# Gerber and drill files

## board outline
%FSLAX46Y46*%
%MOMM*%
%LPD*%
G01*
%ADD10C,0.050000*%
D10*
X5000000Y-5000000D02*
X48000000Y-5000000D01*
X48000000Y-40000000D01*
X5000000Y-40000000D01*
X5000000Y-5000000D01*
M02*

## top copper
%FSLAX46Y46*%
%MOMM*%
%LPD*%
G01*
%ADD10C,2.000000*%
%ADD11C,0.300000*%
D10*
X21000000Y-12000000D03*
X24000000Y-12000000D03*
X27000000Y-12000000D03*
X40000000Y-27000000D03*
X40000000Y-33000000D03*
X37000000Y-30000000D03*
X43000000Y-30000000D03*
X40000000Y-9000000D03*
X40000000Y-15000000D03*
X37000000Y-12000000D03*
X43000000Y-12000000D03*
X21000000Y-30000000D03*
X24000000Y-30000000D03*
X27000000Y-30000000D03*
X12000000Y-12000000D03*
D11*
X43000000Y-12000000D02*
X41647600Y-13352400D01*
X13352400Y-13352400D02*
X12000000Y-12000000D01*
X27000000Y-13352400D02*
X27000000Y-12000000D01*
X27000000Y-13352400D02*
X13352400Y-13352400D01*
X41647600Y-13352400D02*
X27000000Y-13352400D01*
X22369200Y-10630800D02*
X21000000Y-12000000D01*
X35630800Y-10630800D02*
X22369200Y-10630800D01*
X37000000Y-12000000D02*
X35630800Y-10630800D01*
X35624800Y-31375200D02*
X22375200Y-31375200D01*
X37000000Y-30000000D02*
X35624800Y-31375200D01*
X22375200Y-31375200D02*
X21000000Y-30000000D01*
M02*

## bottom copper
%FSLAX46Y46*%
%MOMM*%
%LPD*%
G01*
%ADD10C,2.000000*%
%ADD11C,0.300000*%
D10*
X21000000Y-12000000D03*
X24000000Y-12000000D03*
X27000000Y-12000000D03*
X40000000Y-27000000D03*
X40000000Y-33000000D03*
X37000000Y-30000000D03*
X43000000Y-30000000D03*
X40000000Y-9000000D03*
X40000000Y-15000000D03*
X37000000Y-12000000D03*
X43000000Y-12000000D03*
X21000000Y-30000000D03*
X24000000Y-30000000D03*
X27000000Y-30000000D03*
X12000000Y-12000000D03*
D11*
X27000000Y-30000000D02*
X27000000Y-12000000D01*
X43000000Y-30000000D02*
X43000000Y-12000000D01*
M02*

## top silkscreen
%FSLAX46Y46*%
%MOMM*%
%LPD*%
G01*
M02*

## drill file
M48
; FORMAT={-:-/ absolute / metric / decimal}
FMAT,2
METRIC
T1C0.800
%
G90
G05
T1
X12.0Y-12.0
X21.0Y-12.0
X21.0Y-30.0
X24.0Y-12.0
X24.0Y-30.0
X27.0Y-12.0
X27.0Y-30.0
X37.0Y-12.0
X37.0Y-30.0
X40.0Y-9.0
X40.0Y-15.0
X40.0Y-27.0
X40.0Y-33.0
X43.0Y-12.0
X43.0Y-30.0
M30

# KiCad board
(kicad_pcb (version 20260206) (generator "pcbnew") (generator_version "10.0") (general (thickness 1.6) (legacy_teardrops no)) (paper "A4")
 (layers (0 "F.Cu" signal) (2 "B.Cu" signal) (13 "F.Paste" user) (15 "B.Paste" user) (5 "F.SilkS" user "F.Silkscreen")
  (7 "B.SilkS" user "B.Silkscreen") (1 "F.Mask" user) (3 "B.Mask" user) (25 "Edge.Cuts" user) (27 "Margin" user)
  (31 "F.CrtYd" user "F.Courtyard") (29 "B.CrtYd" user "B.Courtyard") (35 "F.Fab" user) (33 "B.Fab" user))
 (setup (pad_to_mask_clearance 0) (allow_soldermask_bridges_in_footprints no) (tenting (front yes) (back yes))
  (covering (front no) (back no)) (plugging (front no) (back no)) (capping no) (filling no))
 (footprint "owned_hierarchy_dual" (layer "F.Cu") (at 24 12)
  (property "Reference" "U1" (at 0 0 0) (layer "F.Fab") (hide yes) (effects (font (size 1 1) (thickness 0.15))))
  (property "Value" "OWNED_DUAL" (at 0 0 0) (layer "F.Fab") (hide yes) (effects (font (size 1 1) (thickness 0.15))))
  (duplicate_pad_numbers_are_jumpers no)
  (pad "1" thru_hole circle (at -3 0) (size 2 2) (drill 0.8) (layers "*.Cu" "*.Mask") (remove_unused_layers no) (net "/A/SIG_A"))
  (pad "2" thru_hole circle (at 0 0) (size 2 2) (drill 0.8) (layers "*.Cu" "*.Mask") (remove_unused_layers no) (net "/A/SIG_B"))
  (pad "3" thru_hole circle (at 3 0) (size 2 2) (drill 0.8) (layers "*.Cu" "*.Mask") (remove_unused_layers no) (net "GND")))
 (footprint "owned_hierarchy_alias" (layer "F.Cu") (at 40 30)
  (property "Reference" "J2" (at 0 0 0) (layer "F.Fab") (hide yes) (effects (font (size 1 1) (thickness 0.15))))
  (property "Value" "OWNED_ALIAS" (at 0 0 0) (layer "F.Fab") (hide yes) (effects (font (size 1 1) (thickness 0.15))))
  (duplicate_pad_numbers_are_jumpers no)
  (pad "MP" thru_hole circle (at 0 -3) (size 2 2) (drill 0.8) (layers "*.Cu" "*.Mask") (remove_unused_layers no))
  (pad "MP" thru_hole circle (at 0 3) (size 2 2) (drill 0.8) (layers "*.Cu" "*.Mask") (remove_unused_layers no))
  (pad "R" thru_hole circle (at -3 0) (size 2 2) (drill 0.8) (layers "*.Cu" "*.Mask") (remove_unused_layers no) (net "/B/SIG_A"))
  (pad "T" thru_hole circle (at 3 0) (size 2 2) (drill 0.8) (layers "*.Cu" "*.Mask") (remove_unused_layers no) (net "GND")))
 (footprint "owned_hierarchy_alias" (layer "F.Cu") (at 40 12)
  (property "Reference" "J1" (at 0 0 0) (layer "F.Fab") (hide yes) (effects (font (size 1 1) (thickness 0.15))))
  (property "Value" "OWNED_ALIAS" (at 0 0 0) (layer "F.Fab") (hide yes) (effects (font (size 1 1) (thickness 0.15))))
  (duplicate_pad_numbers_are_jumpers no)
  (pad "MP" thru_hole circle (at 0 -3) (size 2 2) (drill 0.8) (layers "*.Cu" "*.Mask") (remove_unused_layers no))
  (pad "MP" thru_hole circle (at 0 3) (size 2 2) (drill 0.8) (layers "*.Cu" "*.Mask") (remove_unused_layers no))
  (pad "R" thru_hole circle (at -3 0) (size 2 2) (drill 0.8) (layers "*.Cu" "*.Mask") (remove_unused_layers no) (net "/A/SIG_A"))
  (pad "T" thru_hole circle (at 3 0) (size 2 2) (drill 0.8) (layers "*.Cu" "*.Mask") (remove_unused_layers no) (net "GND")))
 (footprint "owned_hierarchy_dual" (layer "F.Cu") (at 24 30)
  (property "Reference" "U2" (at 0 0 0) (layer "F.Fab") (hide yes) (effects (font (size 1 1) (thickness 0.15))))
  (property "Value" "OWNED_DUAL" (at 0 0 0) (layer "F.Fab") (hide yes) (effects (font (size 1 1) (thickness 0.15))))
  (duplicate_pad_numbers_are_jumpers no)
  (pad "1" thru_hole circle (at -3 0) (size 2 2) (drill 0.8) (layers "*.Cu" "*.Mask") (remove_unused_layers no) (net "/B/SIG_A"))
  (pad "2" thru_hole circle (at 0 0) (size 2 2) (drill 0.8) (layers "*.Cu" "*.Mask") (remove_unused_layers no) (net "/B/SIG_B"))
  (pad "3" thru_hole circle (at 3 0) (size 2 2) (drill 0.8) (layers "*.Cu" "*.Mask") (remove_unused_layers no) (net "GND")))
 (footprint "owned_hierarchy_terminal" (layer "F.Cu") (at 12 12)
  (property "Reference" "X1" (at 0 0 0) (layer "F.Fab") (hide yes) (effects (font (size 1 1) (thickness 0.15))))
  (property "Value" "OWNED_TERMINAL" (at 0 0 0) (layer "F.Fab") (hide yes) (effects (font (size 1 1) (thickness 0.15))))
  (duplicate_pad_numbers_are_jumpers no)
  (pad "1" thru_hole circle (at 0 0) (size 2 2) (drill 0.8) (layers "*.Cu" "*.Mask") (remove_unused_layers no) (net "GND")))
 (gr_rect (start 5 5) (end 48 40) (stroke (width 0.05) (type default)) (fill no) (layer "Edge.Cuts"))
 (segment (start 43 12) (end 41.6476 13.3524) (width 0.3) (layer "F.Cu") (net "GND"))
 (segment (start 13.3524 13.3524) (end 12 12) (width 0.3) (layer "F.Cu") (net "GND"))
 (segment (start 27 13.3524) (end 27 12) (width 0.3) (layer "F.Cu") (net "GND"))
 (segment (start 27 13.3524) (end 13.3524 13.3524) (width 0.3) (layer "F.Cu") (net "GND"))
 (segment (start 41.6476 13.3524) (end 27 13.3524) (width 0.3) (layer "F.Cu") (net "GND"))
 (segment (start 27 30) (end 27 12) (width 0.3) (layer "B.Cu") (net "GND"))
 (segment (start 43 30) (end 43 12) (width 0.3) (layer "B.Cu") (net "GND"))
 (segment (start 22.3692 10.6308) (end 21 12) (width 0.3) (layer "F.Cu") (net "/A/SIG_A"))
 (segment (start 35.6308 10.6308) (end 22.3692 10.6308) (width 0.3) (layer "F.Cu") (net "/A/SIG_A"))
 (segment (start 37 12) (end 35.6308 10.6308) (width 0.3) (layer "F.Cu") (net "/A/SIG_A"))
 (segment (start 35.6248 31.3752) (end 22.3752 31.3752) (width 0.3) (layer "F.Cu") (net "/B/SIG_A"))
 (segment (start 37 30) (end 35.6248 31.3752) (width 0.3) (layer "F.Cu") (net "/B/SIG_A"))
 (segment (start 22.3752 31.3752) (end 21 30) (width 0.3) (layer "F.Cu") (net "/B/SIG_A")))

